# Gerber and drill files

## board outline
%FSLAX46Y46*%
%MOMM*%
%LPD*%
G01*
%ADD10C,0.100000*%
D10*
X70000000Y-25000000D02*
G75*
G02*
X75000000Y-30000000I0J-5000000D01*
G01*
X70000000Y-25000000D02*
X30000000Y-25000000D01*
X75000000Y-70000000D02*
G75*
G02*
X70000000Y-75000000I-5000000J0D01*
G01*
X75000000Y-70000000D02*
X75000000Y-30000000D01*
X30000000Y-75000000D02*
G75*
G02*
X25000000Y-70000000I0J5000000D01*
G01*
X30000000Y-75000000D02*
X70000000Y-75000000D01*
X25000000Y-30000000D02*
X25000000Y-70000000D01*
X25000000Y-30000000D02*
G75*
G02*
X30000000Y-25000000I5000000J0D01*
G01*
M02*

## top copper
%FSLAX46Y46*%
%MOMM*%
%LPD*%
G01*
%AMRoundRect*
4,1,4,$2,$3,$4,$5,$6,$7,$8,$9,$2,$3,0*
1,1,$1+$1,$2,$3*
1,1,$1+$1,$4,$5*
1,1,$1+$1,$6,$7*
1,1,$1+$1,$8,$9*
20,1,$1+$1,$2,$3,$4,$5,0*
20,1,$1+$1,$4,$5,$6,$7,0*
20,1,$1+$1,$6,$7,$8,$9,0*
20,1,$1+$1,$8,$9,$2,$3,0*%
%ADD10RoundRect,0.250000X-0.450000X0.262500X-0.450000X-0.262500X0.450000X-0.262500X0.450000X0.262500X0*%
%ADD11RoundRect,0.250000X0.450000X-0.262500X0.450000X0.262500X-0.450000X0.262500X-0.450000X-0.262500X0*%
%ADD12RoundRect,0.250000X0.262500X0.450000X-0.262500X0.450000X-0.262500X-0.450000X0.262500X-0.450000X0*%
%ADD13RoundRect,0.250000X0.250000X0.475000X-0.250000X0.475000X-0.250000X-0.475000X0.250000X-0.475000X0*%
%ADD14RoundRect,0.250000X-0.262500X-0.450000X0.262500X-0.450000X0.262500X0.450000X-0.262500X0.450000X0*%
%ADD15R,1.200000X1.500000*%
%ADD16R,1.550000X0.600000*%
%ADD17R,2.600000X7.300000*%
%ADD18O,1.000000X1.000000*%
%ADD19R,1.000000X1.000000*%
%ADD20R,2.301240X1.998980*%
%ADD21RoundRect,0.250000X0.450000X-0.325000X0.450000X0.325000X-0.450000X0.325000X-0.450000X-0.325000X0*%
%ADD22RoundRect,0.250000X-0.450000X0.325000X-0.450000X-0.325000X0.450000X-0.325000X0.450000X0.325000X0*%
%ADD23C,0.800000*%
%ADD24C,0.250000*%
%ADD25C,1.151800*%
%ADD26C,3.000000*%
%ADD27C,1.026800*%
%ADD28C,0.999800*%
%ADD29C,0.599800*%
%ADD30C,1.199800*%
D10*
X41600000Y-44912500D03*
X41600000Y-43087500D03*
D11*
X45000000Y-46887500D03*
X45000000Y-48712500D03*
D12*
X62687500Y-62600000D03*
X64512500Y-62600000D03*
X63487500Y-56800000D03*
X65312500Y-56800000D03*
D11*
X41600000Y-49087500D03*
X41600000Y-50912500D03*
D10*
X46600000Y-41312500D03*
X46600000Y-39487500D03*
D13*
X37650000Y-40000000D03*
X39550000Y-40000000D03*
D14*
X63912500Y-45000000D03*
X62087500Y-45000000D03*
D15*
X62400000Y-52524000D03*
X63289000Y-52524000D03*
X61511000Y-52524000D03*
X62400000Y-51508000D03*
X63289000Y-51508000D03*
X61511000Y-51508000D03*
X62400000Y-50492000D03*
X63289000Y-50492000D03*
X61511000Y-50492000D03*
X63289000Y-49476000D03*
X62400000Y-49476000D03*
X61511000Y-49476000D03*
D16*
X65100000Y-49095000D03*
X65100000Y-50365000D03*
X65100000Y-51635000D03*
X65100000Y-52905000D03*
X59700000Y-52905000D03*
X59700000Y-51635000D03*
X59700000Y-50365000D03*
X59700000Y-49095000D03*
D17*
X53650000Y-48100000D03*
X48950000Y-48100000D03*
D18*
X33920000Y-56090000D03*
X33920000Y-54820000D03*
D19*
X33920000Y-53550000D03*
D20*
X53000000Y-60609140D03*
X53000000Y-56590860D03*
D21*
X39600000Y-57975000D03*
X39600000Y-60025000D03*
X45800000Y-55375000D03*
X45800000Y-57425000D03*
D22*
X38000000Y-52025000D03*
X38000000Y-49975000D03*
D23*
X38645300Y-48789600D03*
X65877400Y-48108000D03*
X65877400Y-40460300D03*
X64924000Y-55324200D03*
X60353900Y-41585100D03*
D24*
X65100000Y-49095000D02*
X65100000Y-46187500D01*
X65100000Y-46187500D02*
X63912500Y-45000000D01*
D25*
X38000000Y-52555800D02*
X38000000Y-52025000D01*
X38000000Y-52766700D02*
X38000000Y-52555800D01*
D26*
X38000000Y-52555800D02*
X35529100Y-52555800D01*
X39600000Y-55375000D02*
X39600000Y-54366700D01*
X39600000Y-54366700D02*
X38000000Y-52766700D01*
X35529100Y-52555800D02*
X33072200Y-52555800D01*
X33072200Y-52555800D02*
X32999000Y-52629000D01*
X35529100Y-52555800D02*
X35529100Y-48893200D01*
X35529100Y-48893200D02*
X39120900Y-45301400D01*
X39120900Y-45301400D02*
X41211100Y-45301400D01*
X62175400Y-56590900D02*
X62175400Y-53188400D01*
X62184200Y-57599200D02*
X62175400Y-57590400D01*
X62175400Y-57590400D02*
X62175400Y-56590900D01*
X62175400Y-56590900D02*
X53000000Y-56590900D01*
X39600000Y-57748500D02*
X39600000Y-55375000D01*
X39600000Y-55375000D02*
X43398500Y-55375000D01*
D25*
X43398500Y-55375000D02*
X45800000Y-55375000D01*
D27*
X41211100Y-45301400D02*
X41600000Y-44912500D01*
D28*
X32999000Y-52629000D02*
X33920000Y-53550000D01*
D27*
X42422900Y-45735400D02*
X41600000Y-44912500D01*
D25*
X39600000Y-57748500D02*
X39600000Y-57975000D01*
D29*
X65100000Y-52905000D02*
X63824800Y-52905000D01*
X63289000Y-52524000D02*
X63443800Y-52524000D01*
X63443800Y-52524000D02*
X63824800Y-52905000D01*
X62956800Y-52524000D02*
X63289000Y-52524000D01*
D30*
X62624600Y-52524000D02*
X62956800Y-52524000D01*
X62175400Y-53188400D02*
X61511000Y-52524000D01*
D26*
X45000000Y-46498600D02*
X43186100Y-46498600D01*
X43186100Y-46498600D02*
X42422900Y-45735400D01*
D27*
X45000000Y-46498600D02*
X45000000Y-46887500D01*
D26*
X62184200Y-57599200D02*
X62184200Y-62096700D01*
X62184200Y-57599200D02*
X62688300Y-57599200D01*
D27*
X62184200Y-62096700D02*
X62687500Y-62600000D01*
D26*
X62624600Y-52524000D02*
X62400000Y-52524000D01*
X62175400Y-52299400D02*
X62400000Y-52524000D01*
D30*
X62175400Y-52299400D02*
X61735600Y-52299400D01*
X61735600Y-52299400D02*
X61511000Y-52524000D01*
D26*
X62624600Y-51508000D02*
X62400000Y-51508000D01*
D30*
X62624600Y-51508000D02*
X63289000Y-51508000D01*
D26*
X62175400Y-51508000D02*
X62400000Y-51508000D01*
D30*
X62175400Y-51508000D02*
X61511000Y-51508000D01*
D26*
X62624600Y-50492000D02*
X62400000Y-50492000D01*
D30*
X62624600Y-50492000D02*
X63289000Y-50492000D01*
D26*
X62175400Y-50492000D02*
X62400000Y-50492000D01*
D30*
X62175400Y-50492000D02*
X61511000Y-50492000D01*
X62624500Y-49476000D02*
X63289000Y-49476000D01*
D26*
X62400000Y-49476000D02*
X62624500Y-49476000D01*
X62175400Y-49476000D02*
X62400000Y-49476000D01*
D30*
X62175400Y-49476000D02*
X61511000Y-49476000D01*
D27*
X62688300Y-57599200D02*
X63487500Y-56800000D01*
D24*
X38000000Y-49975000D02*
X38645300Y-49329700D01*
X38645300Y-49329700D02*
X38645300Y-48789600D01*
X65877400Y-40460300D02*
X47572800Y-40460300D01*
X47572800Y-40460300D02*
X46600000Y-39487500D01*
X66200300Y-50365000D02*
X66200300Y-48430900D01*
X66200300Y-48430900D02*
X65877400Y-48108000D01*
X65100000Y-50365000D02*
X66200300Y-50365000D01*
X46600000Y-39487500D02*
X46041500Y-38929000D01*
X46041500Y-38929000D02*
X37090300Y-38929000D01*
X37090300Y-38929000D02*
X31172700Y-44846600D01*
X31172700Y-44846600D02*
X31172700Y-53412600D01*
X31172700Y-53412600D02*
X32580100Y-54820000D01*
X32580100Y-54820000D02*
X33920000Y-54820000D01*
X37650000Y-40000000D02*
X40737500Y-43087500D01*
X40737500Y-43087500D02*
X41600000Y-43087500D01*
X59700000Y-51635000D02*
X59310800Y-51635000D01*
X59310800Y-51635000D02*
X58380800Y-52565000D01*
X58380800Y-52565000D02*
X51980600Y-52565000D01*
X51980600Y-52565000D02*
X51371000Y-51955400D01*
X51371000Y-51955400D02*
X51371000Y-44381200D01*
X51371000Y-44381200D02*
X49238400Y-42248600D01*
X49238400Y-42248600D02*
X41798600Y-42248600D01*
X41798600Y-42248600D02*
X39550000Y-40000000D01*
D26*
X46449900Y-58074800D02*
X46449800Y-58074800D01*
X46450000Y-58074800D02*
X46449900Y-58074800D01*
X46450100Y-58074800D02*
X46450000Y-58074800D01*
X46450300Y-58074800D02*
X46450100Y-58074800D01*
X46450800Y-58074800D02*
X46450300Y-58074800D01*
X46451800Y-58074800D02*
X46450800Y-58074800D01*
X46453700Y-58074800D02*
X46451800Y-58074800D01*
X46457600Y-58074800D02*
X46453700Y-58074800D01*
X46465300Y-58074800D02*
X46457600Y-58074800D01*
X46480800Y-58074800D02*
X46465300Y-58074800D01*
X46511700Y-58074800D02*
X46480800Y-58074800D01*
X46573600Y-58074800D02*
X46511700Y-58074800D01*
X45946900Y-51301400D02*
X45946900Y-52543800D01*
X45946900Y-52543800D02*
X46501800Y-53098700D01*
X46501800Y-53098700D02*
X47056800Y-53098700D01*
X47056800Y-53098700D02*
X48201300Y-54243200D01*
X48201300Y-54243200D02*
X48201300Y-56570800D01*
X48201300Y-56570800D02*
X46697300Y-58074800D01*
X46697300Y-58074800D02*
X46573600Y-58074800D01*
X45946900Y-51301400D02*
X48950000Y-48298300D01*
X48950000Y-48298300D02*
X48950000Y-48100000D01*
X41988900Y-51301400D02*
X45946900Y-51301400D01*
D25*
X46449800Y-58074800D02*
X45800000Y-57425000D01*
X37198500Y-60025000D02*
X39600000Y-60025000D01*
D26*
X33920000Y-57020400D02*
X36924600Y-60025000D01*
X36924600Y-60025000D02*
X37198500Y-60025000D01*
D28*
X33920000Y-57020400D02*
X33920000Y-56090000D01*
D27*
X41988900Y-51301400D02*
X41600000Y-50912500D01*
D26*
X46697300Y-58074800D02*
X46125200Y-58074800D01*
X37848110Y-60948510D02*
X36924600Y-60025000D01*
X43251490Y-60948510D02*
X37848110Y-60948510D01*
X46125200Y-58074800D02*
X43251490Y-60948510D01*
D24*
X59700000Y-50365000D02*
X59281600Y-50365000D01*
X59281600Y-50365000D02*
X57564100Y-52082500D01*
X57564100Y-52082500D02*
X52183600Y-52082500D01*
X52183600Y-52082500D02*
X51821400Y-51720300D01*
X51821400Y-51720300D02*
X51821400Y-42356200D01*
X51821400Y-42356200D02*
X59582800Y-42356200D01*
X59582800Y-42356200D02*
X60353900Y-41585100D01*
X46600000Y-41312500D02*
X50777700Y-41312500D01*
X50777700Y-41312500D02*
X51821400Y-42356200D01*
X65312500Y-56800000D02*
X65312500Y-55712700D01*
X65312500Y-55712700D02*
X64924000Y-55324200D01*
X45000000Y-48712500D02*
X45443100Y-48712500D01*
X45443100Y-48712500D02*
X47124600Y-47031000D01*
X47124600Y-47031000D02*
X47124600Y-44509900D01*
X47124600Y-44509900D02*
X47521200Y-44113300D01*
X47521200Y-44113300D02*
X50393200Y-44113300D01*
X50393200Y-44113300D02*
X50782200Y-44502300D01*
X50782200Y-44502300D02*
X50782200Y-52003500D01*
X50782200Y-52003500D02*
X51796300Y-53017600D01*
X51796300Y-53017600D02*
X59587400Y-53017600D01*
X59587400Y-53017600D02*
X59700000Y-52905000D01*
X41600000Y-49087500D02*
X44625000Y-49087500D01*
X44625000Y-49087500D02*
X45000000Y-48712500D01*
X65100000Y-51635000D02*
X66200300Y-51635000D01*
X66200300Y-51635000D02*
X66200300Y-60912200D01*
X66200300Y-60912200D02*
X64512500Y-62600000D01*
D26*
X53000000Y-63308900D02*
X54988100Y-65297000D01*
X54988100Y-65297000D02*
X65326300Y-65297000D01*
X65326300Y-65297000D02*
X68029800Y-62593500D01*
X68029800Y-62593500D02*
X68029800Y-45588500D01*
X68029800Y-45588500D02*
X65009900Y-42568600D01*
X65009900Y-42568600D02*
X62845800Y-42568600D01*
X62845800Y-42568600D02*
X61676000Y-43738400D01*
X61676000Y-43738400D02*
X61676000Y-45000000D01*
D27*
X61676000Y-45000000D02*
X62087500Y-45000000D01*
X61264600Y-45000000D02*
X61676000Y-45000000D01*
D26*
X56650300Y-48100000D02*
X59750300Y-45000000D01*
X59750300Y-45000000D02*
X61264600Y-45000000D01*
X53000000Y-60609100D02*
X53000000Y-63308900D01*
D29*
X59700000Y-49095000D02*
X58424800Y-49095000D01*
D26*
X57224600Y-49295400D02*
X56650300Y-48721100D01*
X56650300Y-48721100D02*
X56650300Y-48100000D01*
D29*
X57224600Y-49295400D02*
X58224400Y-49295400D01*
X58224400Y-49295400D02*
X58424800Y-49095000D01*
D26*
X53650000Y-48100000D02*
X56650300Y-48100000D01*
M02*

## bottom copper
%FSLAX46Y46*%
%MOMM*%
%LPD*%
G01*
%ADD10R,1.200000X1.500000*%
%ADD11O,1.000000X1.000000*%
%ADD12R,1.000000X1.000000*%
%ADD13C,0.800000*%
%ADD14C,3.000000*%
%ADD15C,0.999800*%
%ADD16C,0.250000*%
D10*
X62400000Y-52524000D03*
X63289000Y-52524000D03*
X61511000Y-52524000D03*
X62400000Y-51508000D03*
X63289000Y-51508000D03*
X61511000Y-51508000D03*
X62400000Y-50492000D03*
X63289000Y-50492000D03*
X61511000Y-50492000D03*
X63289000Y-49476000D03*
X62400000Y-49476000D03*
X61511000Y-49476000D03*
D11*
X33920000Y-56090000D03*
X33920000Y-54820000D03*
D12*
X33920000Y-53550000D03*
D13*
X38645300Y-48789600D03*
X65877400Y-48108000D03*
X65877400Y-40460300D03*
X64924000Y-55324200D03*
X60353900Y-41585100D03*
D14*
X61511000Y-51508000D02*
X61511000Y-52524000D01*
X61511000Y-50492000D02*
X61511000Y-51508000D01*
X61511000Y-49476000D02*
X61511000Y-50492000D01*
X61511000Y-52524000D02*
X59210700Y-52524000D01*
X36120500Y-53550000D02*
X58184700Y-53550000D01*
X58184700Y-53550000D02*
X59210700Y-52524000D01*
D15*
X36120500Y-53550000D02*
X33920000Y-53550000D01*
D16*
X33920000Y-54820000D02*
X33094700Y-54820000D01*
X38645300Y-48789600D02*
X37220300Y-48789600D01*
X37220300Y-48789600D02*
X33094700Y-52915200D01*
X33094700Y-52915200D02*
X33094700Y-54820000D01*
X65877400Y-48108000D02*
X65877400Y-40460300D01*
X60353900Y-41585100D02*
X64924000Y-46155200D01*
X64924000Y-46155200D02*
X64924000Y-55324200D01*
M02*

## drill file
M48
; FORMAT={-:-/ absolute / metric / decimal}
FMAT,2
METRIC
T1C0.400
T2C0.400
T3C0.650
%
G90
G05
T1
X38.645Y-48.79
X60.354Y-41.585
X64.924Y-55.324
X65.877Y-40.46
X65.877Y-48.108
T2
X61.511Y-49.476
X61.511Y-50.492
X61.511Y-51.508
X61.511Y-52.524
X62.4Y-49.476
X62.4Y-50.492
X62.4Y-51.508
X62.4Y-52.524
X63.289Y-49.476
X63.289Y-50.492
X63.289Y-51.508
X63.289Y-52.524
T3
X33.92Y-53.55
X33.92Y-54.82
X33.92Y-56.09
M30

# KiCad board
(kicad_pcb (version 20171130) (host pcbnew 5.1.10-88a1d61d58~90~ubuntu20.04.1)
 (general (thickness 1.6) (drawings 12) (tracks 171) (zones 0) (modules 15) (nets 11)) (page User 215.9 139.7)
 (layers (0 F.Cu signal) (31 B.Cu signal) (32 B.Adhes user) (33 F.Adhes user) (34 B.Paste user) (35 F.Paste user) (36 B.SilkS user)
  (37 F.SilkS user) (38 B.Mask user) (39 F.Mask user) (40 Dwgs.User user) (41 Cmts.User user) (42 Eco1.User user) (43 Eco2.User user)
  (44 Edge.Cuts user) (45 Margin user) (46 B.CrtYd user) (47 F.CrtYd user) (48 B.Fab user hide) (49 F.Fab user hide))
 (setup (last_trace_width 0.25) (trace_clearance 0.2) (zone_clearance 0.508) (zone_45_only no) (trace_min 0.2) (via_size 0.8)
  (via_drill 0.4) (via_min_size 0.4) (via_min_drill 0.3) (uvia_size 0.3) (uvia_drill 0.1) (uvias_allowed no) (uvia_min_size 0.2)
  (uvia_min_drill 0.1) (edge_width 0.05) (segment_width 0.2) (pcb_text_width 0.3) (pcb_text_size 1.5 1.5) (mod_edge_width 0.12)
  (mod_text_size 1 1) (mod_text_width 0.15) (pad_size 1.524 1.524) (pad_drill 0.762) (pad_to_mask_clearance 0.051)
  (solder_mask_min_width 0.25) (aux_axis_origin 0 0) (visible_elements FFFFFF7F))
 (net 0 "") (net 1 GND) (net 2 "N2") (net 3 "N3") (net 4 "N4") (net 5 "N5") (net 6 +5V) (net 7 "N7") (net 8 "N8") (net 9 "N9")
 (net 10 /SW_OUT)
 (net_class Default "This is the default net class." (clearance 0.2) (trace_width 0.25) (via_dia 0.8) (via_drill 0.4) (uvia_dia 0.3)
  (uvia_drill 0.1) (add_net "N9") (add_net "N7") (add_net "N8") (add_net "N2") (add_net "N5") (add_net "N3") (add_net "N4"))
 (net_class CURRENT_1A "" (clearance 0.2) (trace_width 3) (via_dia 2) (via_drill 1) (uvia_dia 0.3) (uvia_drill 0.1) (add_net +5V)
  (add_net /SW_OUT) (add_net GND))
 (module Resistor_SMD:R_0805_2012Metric (layer F.Cu) (at 41.6 44 270)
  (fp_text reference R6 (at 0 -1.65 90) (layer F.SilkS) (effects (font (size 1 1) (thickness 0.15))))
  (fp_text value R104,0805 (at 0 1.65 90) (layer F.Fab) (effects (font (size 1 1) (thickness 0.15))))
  (pad 2 smd roundrect (at 0.9125 0 270) (size 1.025 1.4) (layers F.Cu F.Paste F.Mask) (roundrect_rratio 0.243902) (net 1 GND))
  (pad 1 smd roundrect (at -0.9125 0 270) (size 1.025 1.4) (layers F.Cu F.Paste F.Mask) (roundrect_rratio 0.243902) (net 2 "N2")))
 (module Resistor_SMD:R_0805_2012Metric (layer F.Cu) (at 45 47.8 90)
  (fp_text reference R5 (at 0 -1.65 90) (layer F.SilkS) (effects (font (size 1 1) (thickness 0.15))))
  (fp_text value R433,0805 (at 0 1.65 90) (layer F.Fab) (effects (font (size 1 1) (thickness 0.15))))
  (pad 2 smd roundrect (at 0.9125 0 90) (size 1.025 1.4) (layers F.Cu F.Paste F.Mask) (roundrect_rratio 0.243902) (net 1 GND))
  (pad 1 smd roundrect (at -0.9125 0 90) (size 1.025 1.4) (layers F.Cu F.Paste F.Mask) (roundrect_rratio 0.243902) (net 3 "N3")))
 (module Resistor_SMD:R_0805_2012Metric (layer F.Cu) (at 63.6 62.6 180)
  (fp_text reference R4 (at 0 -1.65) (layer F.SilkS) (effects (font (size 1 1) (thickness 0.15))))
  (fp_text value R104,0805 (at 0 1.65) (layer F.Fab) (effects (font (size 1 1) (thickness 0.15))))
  (pad 2 smd roundrect (at 0.9125 0 180) (size 1.025 1.4) (layers F.Cu F.Paste F.Mask) (roundrect_rratio 0.243902) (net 1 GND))
  (pad 1 smd roundrect (at -0.9125 0 180) (size 1.025 1.4) (layers F.Cu F.Paste F.Mask) (roundrect_rratio 0.243902) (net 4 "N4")))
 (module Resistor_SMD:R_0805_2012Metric (layer F.Cu) (at 64.4 56.8 180)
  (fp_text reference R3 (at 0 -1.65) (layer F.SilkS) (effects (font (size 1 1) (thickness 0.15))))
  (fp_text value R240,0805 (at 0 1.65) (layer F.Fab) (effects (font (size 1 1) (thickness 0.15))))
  (pad 2 smd roundrect (at 0.9125 0 180) (size 1.025 1.4) (layers F.Cu F.Paste F.Mask) (roundrect_rratio 0.243902) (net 1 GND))
  (pad 1 smd roundrect (at -0.9125 0 180) (size 1.025 1.4) (layers F.Cu F.Paste F.Mask) (roundrect_rratio 0.243902) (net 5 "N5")))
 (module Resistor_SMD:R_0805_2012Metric (layer F.Cu) (at 41.6 50 90)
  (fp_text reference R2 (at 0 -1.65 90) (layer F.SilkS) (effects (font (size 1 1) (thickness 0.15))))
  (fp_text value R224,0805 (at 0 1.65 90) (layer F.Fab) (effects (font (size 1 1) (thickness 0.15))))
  (pad 2 smd roundrect (at 0.9125 0 90) (size 1.025 1.4) (layers F.Cu F.Paste F.Mask) (roundrect_rratio 0.243902) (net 3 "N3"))
  (pad 1 smd roundrect (at -0.9125 0 90) (size 1.025 1.4) (layers F.Cu F.Paste F.Mask) (roundrect_rratio 0.243902) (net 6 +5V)))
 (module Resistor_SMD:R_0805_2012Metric (layer F.Cu) (at 46.6 40.4 270)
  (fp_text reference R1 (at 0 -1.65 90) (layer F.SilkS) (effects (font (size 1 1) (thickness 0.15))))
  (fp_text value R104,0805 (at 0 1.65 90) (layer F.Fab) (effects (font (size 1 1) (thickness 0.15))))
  (pad 2 smd roundrect (at 0.9125 0 270) (size 1.025 1.4) (layers F.Cu F.Paste F.Mask) (roundrect_rratio 0.243902) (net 5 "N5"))
  (pad 1 smd roundrect (at -0.9125 0 270) (size 1.025 1.4) (layers F.Cu F.Paste F.Mask) (roundrect_rratio 0.243902) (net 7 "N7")))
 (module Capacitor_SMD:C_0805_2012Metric (layer F.Cu) (at 38.6 40 180)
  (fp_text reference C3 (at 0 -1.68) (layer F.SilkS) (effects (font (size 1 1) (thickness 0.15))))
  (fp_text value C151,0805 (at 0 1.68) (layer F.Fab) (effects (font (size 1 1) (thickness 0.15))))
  (pad 2 smd roundrect (at 0.95 0 180) (size 1 1.45) (layers F.Cu F.Paste F.Mask) (roundrect_rratio 0.25) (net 2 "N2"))
  (pad 1 smd roundrect (at -0.95 0 180) (size 1 1.45) (layers F.Cu F.Paste F.Mask) (roundrect_rratio 0.25) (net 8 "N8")))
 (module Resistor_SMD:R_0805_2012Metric (layer F.Cu) (at 63 45)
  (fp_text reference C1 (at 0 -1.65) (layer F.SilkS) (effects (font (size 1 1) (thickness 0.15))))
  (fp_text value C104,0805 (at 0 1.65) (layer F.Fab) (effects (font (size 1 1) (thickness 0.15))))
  (pad 2 smd roundrect (at 0.9125 0) (size 1.025 1.4) (layers F.Cu F.Paste F.Mask) (roundrect_rratio 0.243902) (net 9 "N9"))
  (pad 1 smd roundrect (at -0.9125 0) (size 1.025 1.4) (layers F.Cu F.Paste F.Mask) (roundrect_rratio 0.243902) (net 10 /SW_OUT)))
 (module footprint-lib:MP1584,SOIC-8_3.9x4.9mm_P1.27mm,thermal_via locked (layer F.Cu) (at 62.4 51)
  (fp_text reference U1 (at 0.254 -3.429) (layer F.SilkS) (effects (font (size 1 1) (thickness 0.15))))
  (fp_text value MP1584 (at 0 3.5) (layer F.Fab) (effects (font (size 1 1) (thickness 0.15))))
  (pad G thru_hole rect (at 0 1.524) (size 1.2 1.5) (drill 0.4) (layers *.Cu F.Mask) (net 1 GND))
  (pad G thru_hole rect (at 0.889 1.524) (size 1.2 1.5) (drill 0.4) (layers *.Cu F.Mask) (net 1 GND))
  (pad G thru_hole rect (at -0.889 1.524) (size 1.2 1.5) (drill 0.4) (layers *.Cu F.Mask) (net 1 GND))
  (pad G thru_hole rect (at 0 0.508) (size 1.2 1.5) (drill 0.4) (layers *.Cu F.Mask) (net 1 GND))
  (pad G thru_hole rect (at 0.889 0.508) (size 1.2 1.5) (drill 0.4) (layers *.Cu F.Mask) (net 1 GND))
  (pad G thru_hole rect (at -0.889 0.508) (size 1.2 1.5) (drill 0.4) (layers *.Cu F.Mask) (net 1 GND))
  (pad G thru_hole rect (at 0 -0.508) (size 1.2 1.5) (drill 0.4) (layers *.Cu F.Mask) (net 1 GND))
  (pad G thru_hole rect (at 0.889 -0.508) (size 1.2 1.5) (drill 0.4) (layers *.Cu F.Mask) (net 1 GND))
  (pad G thru_hole rect (at -0.889 -0.508) (size 1.2 1.5) (drill 0.4) (layers *.Cu F.Mask) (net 1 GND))
  (pad G thru_hole rect (at 0.889 -1.524) (size 1.2 1.5) (drill 0.4) (layers *.Cu F.Mask) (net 1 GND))
  (pad G thru_hole rect (at 0 -1.524) (size 1.2 1.5) (drill 0.4) (layers *.Cu F.Mask) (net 1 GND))
  (pad G thru_hole rect (at -0.889 -1.524) (size 1.2 1.5) (drill 0.4) (layers *.Cu F.Mask) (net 1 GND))
  (pad 8 smd rect (at 2.7 -1.905) (size 1.55 0.6) (layers F.Cu F.Paste F.Mask) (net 9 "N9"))
  (pad 7 smd rect (at 2.7 -0.635) (size 1.55 0.6) (layers F.Cu F.Paste F.Mask) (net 7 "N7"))
  (pad 6 smd rect (at 2.7 0.635) (size 1.55 0.6) (layers F.Cu F.Paste F.Mask) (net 4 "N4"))
  (pad 5 smd rect (at 2.7 1.905) (size 1.55 0.6) (layers F.Cu F.Paste F.Mask) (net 1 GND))
  (pad 4 smd rect (at -2.7 1.905) (size 1.55 0.6) (layers F.Cu F.Paste F.Mask) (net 3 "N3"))
  (pad 3 smd rect (at -2.7 0.635) (size 1.55 0.6) (layers F.Cu F.Paste F.Mask) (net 8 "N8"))
  (pad 2 smd rect (at -2.7 -0.635) (size 1.55 0.6) (layers F.Cu F.Paste F.Mask) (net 5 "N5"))
  (pad 1 smd rect (at -2.7 -1.905) (size 1.55 0.6) (layers F.Cu F.Paste F.Mask) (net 10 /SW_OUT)))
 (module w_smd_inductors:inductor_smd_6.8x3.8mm (layer F.Cu) (at 51.3 48.1 270)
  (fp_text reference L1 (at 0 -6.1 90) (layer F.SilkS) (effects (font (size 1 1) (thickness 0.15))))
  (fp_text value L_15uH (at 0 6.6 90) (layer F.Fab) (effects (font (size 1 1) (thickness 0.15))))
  (pad 1 smd rect (at 0 -2.35 270) (size 7.3 2.6) (layers F.Cu F.Paste F.Mask) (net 10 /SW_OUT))
  (pad 2 smd rect (at 0 2.35 270) (size 7.3 2.6) (layers F.Cu F.Paste F.Mask) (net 6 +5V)))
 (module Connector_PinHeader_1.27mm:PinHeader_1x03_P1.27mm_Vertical (layer F.Cu) (at 33.92 53.55)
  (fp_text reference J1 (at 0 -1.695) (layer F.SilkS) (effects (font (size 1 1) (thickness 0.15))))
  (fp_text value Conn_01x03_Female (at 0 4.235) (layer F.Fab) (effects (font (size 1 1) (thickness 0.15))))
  (pad 3 thru_hole oval (at 0 2.54) (size 1 1) (drill 0.65) (layers *.Cu *.Mask) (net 6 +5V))
  (pad 2 thru_hole oval (at 0 1.27) (size 1 1) (drill 0.65) (layers *.Cu *.Mask) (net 7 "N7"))
  (pad 1 thru_hole rect (at 0 0) (size 1 1) (drill 0.65) (layers *.Cu *.Mask) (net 1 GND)))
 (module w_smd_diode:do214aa (layer F.Cu) (at 53 58.6 90)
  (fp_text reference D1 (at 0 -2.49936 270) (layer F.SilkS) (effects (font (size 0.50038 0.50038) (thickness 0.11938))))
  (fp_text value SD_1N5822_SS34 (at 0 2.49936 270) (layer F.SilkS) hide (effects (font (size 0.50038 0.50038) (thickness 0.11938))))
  (pad 1 smd rect (at -2.00914 0 90) (size 1.99898 2.30124) (layers F.Cu F.Paste F.Mask) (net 10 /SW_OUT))
  (pad 2 smd rect (at 2.00914 0 90) (size 1.99898 2.30124) (layers F.Cu F.Paste F.Mask) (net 1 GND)))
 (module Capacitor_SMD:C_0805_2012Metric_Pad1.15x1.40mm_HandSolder (layer F.Cu) (at 39.6 59 90)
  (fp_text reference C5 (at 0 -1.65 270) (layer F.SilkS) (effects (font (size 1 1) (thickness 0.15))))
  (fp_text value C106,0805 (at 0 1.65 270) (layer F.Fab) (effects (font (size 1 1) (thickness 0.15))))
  (pad 2 smd roundrect (at 1.025 0 90) (size 1.15 1.4) (layers F.Cu F.Paste F.Mask) (roundrect_rratio 0.217391) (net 1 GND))
  (pad 1 smd roundrect (at -1.025 0 90) (size 1.15 1.4) (layers F.Cu F.Paste F.Mask) (roundrect_rratio 0.217391) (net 6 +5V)))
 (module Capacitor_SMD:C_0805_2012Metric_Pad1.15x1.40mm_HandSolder (layer F.Cu) (at 45.8 56.4 90)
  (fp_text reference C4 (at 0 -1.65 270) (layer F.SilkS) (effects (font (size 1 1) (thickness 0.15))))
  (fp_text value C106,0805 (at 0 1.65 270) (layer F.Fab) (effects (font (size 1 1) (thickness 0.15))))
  (pad 2 smd roundrect (at 1.025 0 90) (size 1.15 1.4) (layers F.Cu F.Paste F.Mask) (roundrect_rratio 0.217391) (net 1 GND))
  (pad 1 smd roundrect (at -1.025 0 90) (size 1.15 1.4) (layers F.Cu F.Paste F.Mask) (roundrect_rratio 0.217391) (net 6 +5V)))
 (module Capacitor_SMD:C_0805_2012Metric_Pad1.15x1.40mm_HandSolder (layer F.Cu) (at 38 51 270)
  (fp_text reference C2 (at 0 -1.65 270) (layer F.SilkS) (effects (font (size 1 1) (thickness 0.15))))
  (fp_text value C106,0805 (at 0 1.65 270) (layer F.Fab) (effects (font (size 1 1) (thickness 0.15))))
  (pad 2 smd roundrect (at 1.025 0 270) (size 1.15 1.4) (layers F.Cu F.Paste F.Mask) (roundrect_rratio 0.217391) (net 1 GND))
  (pad 1 smd roundrect (at -1.025 0 270) (size 1.15 1.4) (layers F.Cu F.Paste F.Mask) (roundrect_rratio 0.217391) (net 7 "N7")))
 (gr_arc (start 70 30) (end 75 30) (angle -90) (layer Edge.Cuts) (width 0.1))
 (gr_line (start 70 25) (end 30 25) (layer Edge.Cuts) (width 0.1))
 (gr_arc (start 70 70) (end 70 75) (angle -90) (layer Edge.Cuts) (width 0.1))
 (gr_line (start 75 70) (end 75 30) (layer Edge.Cuts) (width 0.1))
 (gr_arc (start 30 70) (end 25 70) (angle -90) (layer Edge.Cuts) (width 0.1))
 (gr_line (start 30 75) (end 70 75) (layer Edge.Cuts) (width 0.1))
 (gr_line (start 25 30) (end 25 70) (layer Edge.Cuts) (width 0.1))
 (gr_arc (start 30 30) (end 30 25) (angle -90) (layer Edge.Cuts) (width 0.1))
 (segment (start 65.1 49.095) (end 65.1 46.1875) (width 0.25) (layer F.Cu) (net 9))
 (segment (start 65.1 46.1875) (end 63.9125 45) (width 0.25) (layer F.Cu) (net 9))
 (segment (start 38 52.5558) (end 38 52.025) (width 1.1518) (layer F.Cu) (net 1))
 (segment (start 38 52.7667) (end 38 52.5558) (width 1.1518) (layer F.Cu) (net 1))
 (segment (start 38 52.5558) (end 35.5291 52.5558) (width 3) (layer F.Cu) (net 1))
 (segment (start 39.6 55.375) (end 39.6 54.3667) (width 3) (layer F.Cu) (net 1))
 (segment (start 39.6 54.3667) (end 38 52.7667) (width 3) (layer F.Cu) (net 1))
 (segment (start 35.5291 52.5558) (end 33.0722 52.5558) (width 3) (layer F.Cu) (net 1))
 (segment (start 33.0722 52.5558) (end 32.999 52.629) (width 3) (layer F.Cu) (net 1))
 (segment (start 35.5291 52.5558) (end 35.5291 48.8932) (width 3) (layer F.Cu) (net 1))
 (segment (start 35.5291 48.8932) (end 39.1209 45.3014) (width 3) (layer F.Cu) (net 1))
 (segment (start 39.1209 45.3014) (end 41.2111 45.3014) (width 3) (layer F.Cu) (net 1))
 (segment (start 62.1754 56.5909) (end 62.1754 53.1884) (width 3) (layer F.Cu) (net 1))
 (segment (start 62.1842 57.5992) (end 62.1754 57.5904) (width 3) (layer F.Cu) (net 1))
 (segment (start 62.1754 57.5904) (end 62.1754 56.5909) (width 3) (layer F.Cu) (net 1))
 (segment (start 62.1754 56.5909) (end 53 56.5909) (width 3) (layer F.Cu) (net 1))
 (segment (start 39.6 57.7485) (end 39.6 55.375) (width 3) (layer F.Cu) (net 1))
 (segment (start 39.6 55.375) (end 43.3985 55.375) (width 3) (layer F.Cu) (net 1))
 (segment (start 43.3985 55.375) (end 45.8 55.375) (width 1.1518) (layer F.Cu) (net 1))
 (segment (start 41.2111 45.3014) (end 41.6 44.9125) (width 1.0268) (layer F.Cu) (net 1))
 (segment (start 32.999 52.629) (end 33.92 53.55) (width 0.9998) (layer F.Cu) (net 1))
 (segment (start 42.4229 45.7354) (end 41.6 44.9125) (width 1.0268) (layer F.Cu) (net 1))
 (segment (start 39.6 57.7485) (end 39.6 57.975) (width 1.1518) (layer F.Cu) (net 1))
 (segment (start 65.1 52.905) (end 63.8248 52.905) (width 0.5998) (layer F.Cu) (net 1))
 (segment (start 63.289 52.524) (end 63.4438 52.524) (width 0.5998) (layer F.Cu) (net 1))
 (segment (start 63.4438 52.524) (end 63.8248 52.905) (width 0.5998) (layer F.Cu) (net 1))
 (segment (start 62.9568 52.524) (end 63.289 52.524) (width 0.5998) (layer F.Cu) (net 1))
 (segment (start 62.6246 52.524) (end 62.9568 52.524) (width 1.1998) (layer F.Cu) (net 1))
 (segment (start 62.1754 53.1884) (end 61.511 52.524) (width 1.1998) (layer F.Cu) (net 1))
 (segment (start 45 46.4986) (end 43.1861 46.4986) (width 3) (layer F.Cu) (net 1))
 (segment (start 43.1861 46.4986) (end 42.4229 45.7354) (width 3) (layer F.Cu) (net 1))
 (segment (start 45 46.4986) (end 45 46.8875) (width 1.0268) (layer F.Cu) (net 1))
 (segment (start 62.1842 57.5992) (end 62.1842 62.0967) (width 3) (layer F.Cu) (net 1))
 (segment (start 62.1842 57.5992) (end 62.6883 57.5992) (width 3) (layer F.Cu) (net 1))
 (segment (start 62.1842 62.0967) (end 62.6875 62.6) (width 1.0268) (layer F.Cu) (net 1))
 (segment (start 62.6246 52.524) (end 62.4 52.524) (width 3) (layer F.Cu) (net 1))
 (segment (start 62.1754 52.2994) (end 62.4 52.524) (width 3) (layer F.Cu) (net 1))
 (segment (start 62.1754 52.2994) (end 61.7356 52.2994) (width 1.1998) (layer F.Cu) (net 1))
 (segment (start 61.7356 52.2994) (end 61.511 52.524) (width 1.1998) (layer F.Cu) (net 1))
 (segment (start 61.511 51.508) (end 61.511 52.524) (width 3) (layer B.Cu) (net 1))
 (segment (start 61.511 50.492) (end 61.511 51.508) (width 3) (layer B.Cu) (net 1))
 (segment (start 62.6246 51.508) (end 62.4 51.508) (width 3) (layer F.Cu) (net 1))
 (segment (start 62.6246 51.508) (end 63.289 51.508) (width 1.1998) (layer F.Cu) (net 1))
 (segment (start 62.1754 51.508) (end 62.4 51.508) (width 3) (layer F.Cu) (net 1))
 (segment (start 62.1754 51.508) (end 61.511 51.508) (width 1.1998) (layer F.Cu) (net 1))
 (segment (start 61.511 49.476) (end 61.511 50.492) (width 3) (layer B.Cu) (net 1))
 (segment (start 62.6246 50.492) (end 62.4 50.492) (width 3) (layer F.Cu) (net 1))
 (segment (start 62.6246 50.492) (end 63.289 50.492) (width 1.1998) (layer F.Cu) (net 1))
 (segment (start 62.1754 50.492) (end 62.4 50.492) (width 3) (layer F.Cu) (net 1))
 (segment (start 62.1754 50.492) (end 61.511 50.492) (width 1.1998) (layer F.Cu) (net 1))
 (segment (start 62.6245 49.476) (end 63.289 49.476) (width 1.1998) (layer F.Cu) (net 1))
 (segment (start 62.4 49.476) (end 62.6245 49.476) (width 3) (layer F.Cu) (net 1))
 (segment (start 62.1754 49.476) (end 62.4 49.476) (width 3) (layer F.Cu) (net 1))
 (segment (start 62.1754 49.476) (end 61.511 49.476) (width 1.1998) (layer F.Cu) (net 1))
 (segment (start 61.511 52.524) (end 59.2107 52.524) (width 3) (layer B.Cu) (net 1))
 (segment (start 36.1205 53.55) (end 58.1847 53.55) (width 3) (layer B.Cu) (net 1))
 (segment (start 58.1847 53.55) (end 59.2107 52.524) (width 3) (layer B.Cu) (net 1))
 (segment (start 36.1205 53.55) (end 33.92 53.55) (width 0.9998) (layer B.Cu) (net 1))
 (segment (start 62.6883 57.5992) (end 63.4875 56.8) (width 1.0268) (layer F.Cu) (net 1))
 (segment (start 33.92 54.82) (end 33.0947 54.82) (width 0.25) (layer B.Cu) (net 7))
 (segment (start 38.6453 48.7896) (end 37.2203 48.7896) (width 0.25) (layer B.Cu) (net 7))
 (segment (start 37.2203 48.7896) (end 33.0947 52.9152) (width 0.25) (layer B.Cu) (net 7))
 (segment (start 33.0947 52.9152) (end 33.0947 54.82) (width 0.25) (layer B.Cu) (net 7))
 (segment (start 38 49.975) (end 38.6453 49.3297) (width 0.25) (layer F.Cu) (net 7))
 (segment (start 38.6453 49.3297) (end 38.6453 48.7896) (width 0.25) (layer F.Cu) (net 7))
 (segment (start 65.8774 40.4603) (end 47.5728 40.4603) (width 0.25) (layer F.Cu) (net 7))
 (segment (start 47.5728 40.4603) (end 46.6 39.4875) (width 0.25) (layer F.Cu) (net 7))
 (segment (start 65.8774 48.108) (end 65.8774 40.4603) (width 0.25) (layer B.Cu) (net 7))
 (segment (start 66.2003 50.365) (end 66.2003 48.4309) (width 0.25) (layer F.Cu) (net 7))
 (segment (start 66.2003 48.4309) (end 65.8774 48.108) (width 0.25) (layer F.Cu) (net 7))
 (segment (start 65.1 50.365) (end 66.2003 50.365) (width 0.25) (layer F.Cu) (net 7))
 (segment (start 46.6 39.4875) (end 46.0415 38.929) (width 0.25) (layer F.Cu) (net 7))
 (segment (start 46.0415 38.929) (end 37.0903 38.929) (width 0.25) (layer F.Cu) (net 7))
 (segment (start 37.0903 38.929) (end 31.1727 44.8466) (width 0.25) (layer F.Cu) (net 7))
 (segment (start 31.1727 44.8466) (end 31.1727 53.4126) (width 0.25) (layer F.Cu) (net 7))
 (segment (start 31.1727 53.4126) (end 32.5801 54.82) (width 0.25) (layer F.Cu) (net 7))
 (segment (start 32.5801 54.82) (end 33.92 54.82) (width 0.25) (layer F.Cu) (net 7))
 (via (at 38.6453 48.7896) (size 0.8) (layers F.Cu B.Cu) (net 7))
 (via (at 65.8774 48.108) (size 0.8) (layers F.Cu B.Cu) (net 7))
 (via (at 65.8774 40.4603) (size 0.8) (layers F.Cu B.Cu) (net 7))
 (segment (start 37.65 40) (end 40.7375 43.0875) (width 0.25) (layer F.Cu) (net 2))
 (segment (start 40.7375 43.0875) (end 41.6 43.0875) (width 0.25) (layer F.Cu) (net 2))
 (segment (start 59.7 51.635) (end 59.3108 51.635) (width 0.25) (layer F.Cu) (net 8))
 (segment (start 59.3108 51.635) (end 58.3808 52.565) (width 0.25) (layer F.Cu) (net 8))
 (segment (start 58.3808 52.565) (end 51.9806 52.565) (width 0.25) (layer F.Cu) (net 8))
 (segment (start 51.9806 52.565) (end 51.371 51.9554) (width 0.25) (layer F.Cu) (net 8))
 (segment (start 51.371 51.9554) (end 51.371 44.3812) (width 0.25) (layer F.Cu) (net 8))
 (segment (start 51.371 44.3812) (end 49.2384 42.2486) (width 0.25) (layer F.Cu) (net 8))
 (segment (start 49.2384 42.2486) (end 41.7986 42.2486) (width 0.25) (layer F.Cu) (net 8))
 (segment (start 41.7986 42.2486) (end 39.55 40) (width 0.25) (layer F.Cu) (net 8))
 (segment (start 46.4499 58.0748) (end 46.4498 58.0748) (width 3) (layer F.Cu) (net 6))
 (segment (start 46.45 58.0748) (end 46.4499 58.0748) (width 3) (layer F.Cu) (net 6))
 (segment (start 46.4501 58.0748) (end 46.45 58.0748) (width 3) (layer F.Cu) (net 6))
 (segment (start 46.4503 58.0748) (end 46.4501 58.0748) (width 3) (layer F.Cu) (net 6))
 (segment (start 46.4508 58.0748) (end 46.4503 58.0748) (width 3) (layer F.Cu) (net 6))
 (segment (start 46.4518 58.0748) (end 46.4508 58.0748) (width 3) (layer F.Cu) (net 6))
 (segment (start 46.4537 58.0748) (end 46.4518 58.0748) (width 3) (layer F.Cu) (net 6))
 (segment (start 46.4576 58.0748) (end 46.4537 58.0748) (width 3) (layer F.Cu) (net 6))
 (segment (start 46.4653 58.0748) (end 46.4576 58.0748) (width 3) (layer F.Cu) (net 6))
 (segment (start 46.4808 58.0748) (end 46.4653 58.0748) (width 3) (layer F.Cu) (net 6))
 (segment (start 46.5117 58.0748) (end 46.4808 58.0748) (width 3) (layer F.Cu) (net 6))
 (segment (start 46.5736 58.0748) (end 46.5117 58.0748) (width 3) (layer F.Cu) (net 6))
 (segment (start 45.9469 51.3014) (end 45.9469 52.5438) (width 3) (layer F.Cu) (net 6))
 (segment (start 45.9469 52.5438) (end 46.5018 53.0987) (width 3) (layer F.Cu) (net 6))
 (segment (start 46.5018 53.0987) (end 47.0568 53.0987) (width 3) (layer F.Cu) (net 6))
 (segment (start 47.0568 53.0987) (end 48.2013 54.2432) (width 3) (layer F.Cu) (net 6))
 (segment (start 48.2013 54.2432) (end 48.2013 56.5708) (width 3) (layer F.Cu) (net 6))
 (segment (start 48.2013 56.5708) (end 46.6973 58.0748) (width 3) (layer F.Cu) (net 6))
 (segment (start 46.6973 58.0748) (end 46.5736 58.0748) (width 3) (layer F.Cu) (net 6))
 (segment (start 45.9469 51.3014) (end 48.95 48.2983) (width 3) (layer F.Cu) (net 6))
 (segment (start 48.95 48.2983) (end 48.95 48.1) (width 3) (layer F.Cu) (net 6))
 (segment (start 41.9889 51.3014) (end 45.9469 51.3014) (width 3) (layer F.Cu) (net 6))
 (segment (start 46.4498 58.0748) (end 45.8 57.425) (width 1.1518) (layer F.Cu) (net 6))
 (segment (start 37.1985 60.025) (end 39.6 60.025) (width 1.1518) (layer F.Cu) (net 6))
 (segment (start 33.92 57.0204) (end 36.9246 60.025) (width 3) (layer F.Cu) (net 6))
 (segment (start 36.9246 60.025) (end 37.1985 60.025) (width 3) (layer F.Cu) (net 6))
 (segment (start 33.92 57.0204) (end 33.92 56.09) (width 0.9998) (layer F.Cu) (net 6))
 (segment (start 41.9889 51.3014) (end 41.6 50.9125) (width 1.0268) (layer F.Cu) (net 6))
 (segment (start 46.6973 58.0748) (end 46.1252 58.0748) (width 3) (layer F.Cu) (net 6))
 (segment (start 37.84811 60.94851) (end 36.9246 60.025) (width 3) (layer F.Cu) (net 6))
 (segment (start 43.25149 60.94851) (end 37.84811 60.94851) (width 3) (layer F.Cu) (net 6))
 (segment (start 46.1252 58.0748) (end 43.25149 60.94851) (width 3) (layer F.Cu) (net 6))
 (segment (start 59.7 50.365) (end 59.2816 50.365) (width 0.25) (layer F.Cu) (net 5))
 (segment (start 59.2816 50.365) (end 57.5641 52.0825) (width 0.25) (layer F.Cu) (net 5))
 (segment (start 57.5641 52.0825) (end 52.1836 52.0825) (width 0.25) (layer F.Cu) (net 5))
 (segment (start 52.1836 52.0825) (end 51.8214 51.7203) (width 0.25) (layer F.Cu) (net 5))
 (segment (start 51.8214 51.7203) (end 51.8214 42.3562) (width 0.25) (layer F.Cu) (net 5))
 (segment (start 51.8214 42.3562) (end 59.5828 42.3562) (width 0.25) (layer F.Cu) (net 5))
 (segment (start 59.5828 42.3562) (end 60.3539 41.5851) (width 0.25) (layer F.Cu) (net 5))
 (segment (start 46.6 41.3125) (end 50.7777 41.3125) (width 0.25) (layer F.Cu) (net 5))
 (segment (start 50.7777 41.3125) (end 51.8214 42.3562) (width 0.25) (layer F.Cu) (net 5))
 (segment (start 65.3125 56.8) (end 65.3125 55.7127) (width 0.25) (layer F.Cu) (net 5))
 (segment (start 65.3125 55.7127) (end 64.924 55.3242) (width 0.25) (layer F.Cu) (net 5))
 (segment (start 60.3539 41.5851) (end 64.924 46.1552) (width 0.25) (layer B.Cu) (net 5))
 (segment (start 64.924 46.1552) (end 64.924 55.3242) (width 0.25) (layer B.Cu) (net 5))
 (via (at 64.924 55.3242) (size 0.8) (layers F.Cu B.Cu) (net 5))
 (via (at 60.3539 41.5851) (size 0.8) (layers F.Cu B.Cu) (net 5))
 (segment (start 45 48.7125) (end 45.4431 48.7125) (width 0.25) (layer F.Cu) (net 3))
 (segment (start 45.4431 48.7125) (end 47.1246 47.031) (width 0.25) (layer F.Cu) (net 3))
 (segment (start 47.1246 47.031) (end 47.1246 44.5099) (width 0.25) (layer F.Cu) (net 3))
 (segment (start 47.1246 44.5099) (end 47.5212 44.1133) (width 0.25) (layer F.Cu) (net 3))
 (segment (start 47.5212 44.1133) (end 50.3932 44.1133) (width 0.25) (layer F.Cu) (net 3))
 (segment (start 50.3932 44.1133) (end 50.7822 44.5023) (width 0.25) (layer F.Cu) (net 3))
 (segment (start 50.7822 44.5023) (end 50.7822 52.0035) (width 0.25) (layer F.Cu) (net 3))
 (segment (start 50.7822 52.0035) (end 51.7963 53.0176) (width 0.25) (layer F.Cu) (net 3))
 (segment (start 51.7963 53.0176) (end 59.5874 53.0176) (width 0.25) (layer F.Cu) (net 3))
 (segment (start 59.5874 53.0176) (end 59.7 52.905) (width 0.25) (layer F.Cu) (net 3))
 (segment (start 41.6 49.0875) (end 44.625 49.0875) (width 0.25) (layer F.Cu) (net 3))
 (segment (start 44.625 49.0875) (end 45 48.7125) (width 0.25) (layer F.Cu) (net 3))
 (segment (start 65.1 51.635) (end 66.2003 51.635) (width 0.25) (layer F.Cu) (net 4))
 (segment (start 66.2003 51.635) (end 66.2003 60.9122) (width 0.25) (layer F.Cu) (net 4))
 (segment (start 66.2003 60.9122) (end 64.5125 62.6) (width 0.25) (layer F.Cu) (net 4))
 (segment (start 53 63.3089) (end 54.9881 65.297) (width 3) (layer F.Cu) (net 10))
 (segment (start 54.9881 65.297) (end 65.3263 65.297) (width 3) (layer F.Cu) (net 10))
 (segment (start 65.3263 65.297) (end 68.0298 62.5935) (width 3) (layer F.Cu) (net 10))
 (segment (start 68.0298 62.5935) (end 68.0298 45.5885) (width 3) (layer F.Cu) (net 10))
 (segment (start 68.0298 45.5885) (end 65.0099 42.5686) (width 3) (layer F.Cu) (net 10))
 (segment (start 65.0099 42.5686) (end 62.8458 42.5686) (width 3) (layer F.Cu) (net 10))
 (segment (start 62.8458 42.5686) (end 61.676 43.7384) (width 3) (layer F.Cu) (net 10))
 (segment (start 61.676 43.7384) (end 61.676 45) (width 3) (layer F.Cu) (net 10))
 (segment (start 61.676 45) (end 62.0875 45) (width 1.0268) (layer F.Cu) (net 10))
 (segment (start 61.2646 45) (end 61.676 45) (width 1.0268) (layer F.Cu) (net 10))
 (segment (start 56.6503 48.1) (end 59.7503 45) (width 3) (layer F.Cu) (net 10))
 (segment (start 59.7503 45) (end 61.2646 45) (width 3) (layer F.Cu) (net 10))
 (segment (start 53 60.6091) (end 53 63.3089) (width 3) (layer F.Cu) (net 10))
 (segment (start 59.7 49.095) (end 58.4248 49.095) (width 0.5998) (layer F.Cu) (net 10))
 (segment (start 57.2246 49.2954) (end 56.6503 48.7211) (width 3) (layer F.Cu) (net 10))
 (segment (start 56.6503 48.7211) (end 56.6503 48.1) (width 3) (layer F.Cu) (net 10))
 (segment (start 57.2246 49.2954) (end 58.2244 49.2954) (width 0.5998) (layer F.Cu) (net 10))
 (segment (start 58.2244 49.2954) (end 58.4248 49.095) (width 0.5998) (layer F.Cu) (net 10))
 (segment (start 53.65 48.1) (end 56.6503 48.1) (width 3) (layer F.Cu) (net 10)))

